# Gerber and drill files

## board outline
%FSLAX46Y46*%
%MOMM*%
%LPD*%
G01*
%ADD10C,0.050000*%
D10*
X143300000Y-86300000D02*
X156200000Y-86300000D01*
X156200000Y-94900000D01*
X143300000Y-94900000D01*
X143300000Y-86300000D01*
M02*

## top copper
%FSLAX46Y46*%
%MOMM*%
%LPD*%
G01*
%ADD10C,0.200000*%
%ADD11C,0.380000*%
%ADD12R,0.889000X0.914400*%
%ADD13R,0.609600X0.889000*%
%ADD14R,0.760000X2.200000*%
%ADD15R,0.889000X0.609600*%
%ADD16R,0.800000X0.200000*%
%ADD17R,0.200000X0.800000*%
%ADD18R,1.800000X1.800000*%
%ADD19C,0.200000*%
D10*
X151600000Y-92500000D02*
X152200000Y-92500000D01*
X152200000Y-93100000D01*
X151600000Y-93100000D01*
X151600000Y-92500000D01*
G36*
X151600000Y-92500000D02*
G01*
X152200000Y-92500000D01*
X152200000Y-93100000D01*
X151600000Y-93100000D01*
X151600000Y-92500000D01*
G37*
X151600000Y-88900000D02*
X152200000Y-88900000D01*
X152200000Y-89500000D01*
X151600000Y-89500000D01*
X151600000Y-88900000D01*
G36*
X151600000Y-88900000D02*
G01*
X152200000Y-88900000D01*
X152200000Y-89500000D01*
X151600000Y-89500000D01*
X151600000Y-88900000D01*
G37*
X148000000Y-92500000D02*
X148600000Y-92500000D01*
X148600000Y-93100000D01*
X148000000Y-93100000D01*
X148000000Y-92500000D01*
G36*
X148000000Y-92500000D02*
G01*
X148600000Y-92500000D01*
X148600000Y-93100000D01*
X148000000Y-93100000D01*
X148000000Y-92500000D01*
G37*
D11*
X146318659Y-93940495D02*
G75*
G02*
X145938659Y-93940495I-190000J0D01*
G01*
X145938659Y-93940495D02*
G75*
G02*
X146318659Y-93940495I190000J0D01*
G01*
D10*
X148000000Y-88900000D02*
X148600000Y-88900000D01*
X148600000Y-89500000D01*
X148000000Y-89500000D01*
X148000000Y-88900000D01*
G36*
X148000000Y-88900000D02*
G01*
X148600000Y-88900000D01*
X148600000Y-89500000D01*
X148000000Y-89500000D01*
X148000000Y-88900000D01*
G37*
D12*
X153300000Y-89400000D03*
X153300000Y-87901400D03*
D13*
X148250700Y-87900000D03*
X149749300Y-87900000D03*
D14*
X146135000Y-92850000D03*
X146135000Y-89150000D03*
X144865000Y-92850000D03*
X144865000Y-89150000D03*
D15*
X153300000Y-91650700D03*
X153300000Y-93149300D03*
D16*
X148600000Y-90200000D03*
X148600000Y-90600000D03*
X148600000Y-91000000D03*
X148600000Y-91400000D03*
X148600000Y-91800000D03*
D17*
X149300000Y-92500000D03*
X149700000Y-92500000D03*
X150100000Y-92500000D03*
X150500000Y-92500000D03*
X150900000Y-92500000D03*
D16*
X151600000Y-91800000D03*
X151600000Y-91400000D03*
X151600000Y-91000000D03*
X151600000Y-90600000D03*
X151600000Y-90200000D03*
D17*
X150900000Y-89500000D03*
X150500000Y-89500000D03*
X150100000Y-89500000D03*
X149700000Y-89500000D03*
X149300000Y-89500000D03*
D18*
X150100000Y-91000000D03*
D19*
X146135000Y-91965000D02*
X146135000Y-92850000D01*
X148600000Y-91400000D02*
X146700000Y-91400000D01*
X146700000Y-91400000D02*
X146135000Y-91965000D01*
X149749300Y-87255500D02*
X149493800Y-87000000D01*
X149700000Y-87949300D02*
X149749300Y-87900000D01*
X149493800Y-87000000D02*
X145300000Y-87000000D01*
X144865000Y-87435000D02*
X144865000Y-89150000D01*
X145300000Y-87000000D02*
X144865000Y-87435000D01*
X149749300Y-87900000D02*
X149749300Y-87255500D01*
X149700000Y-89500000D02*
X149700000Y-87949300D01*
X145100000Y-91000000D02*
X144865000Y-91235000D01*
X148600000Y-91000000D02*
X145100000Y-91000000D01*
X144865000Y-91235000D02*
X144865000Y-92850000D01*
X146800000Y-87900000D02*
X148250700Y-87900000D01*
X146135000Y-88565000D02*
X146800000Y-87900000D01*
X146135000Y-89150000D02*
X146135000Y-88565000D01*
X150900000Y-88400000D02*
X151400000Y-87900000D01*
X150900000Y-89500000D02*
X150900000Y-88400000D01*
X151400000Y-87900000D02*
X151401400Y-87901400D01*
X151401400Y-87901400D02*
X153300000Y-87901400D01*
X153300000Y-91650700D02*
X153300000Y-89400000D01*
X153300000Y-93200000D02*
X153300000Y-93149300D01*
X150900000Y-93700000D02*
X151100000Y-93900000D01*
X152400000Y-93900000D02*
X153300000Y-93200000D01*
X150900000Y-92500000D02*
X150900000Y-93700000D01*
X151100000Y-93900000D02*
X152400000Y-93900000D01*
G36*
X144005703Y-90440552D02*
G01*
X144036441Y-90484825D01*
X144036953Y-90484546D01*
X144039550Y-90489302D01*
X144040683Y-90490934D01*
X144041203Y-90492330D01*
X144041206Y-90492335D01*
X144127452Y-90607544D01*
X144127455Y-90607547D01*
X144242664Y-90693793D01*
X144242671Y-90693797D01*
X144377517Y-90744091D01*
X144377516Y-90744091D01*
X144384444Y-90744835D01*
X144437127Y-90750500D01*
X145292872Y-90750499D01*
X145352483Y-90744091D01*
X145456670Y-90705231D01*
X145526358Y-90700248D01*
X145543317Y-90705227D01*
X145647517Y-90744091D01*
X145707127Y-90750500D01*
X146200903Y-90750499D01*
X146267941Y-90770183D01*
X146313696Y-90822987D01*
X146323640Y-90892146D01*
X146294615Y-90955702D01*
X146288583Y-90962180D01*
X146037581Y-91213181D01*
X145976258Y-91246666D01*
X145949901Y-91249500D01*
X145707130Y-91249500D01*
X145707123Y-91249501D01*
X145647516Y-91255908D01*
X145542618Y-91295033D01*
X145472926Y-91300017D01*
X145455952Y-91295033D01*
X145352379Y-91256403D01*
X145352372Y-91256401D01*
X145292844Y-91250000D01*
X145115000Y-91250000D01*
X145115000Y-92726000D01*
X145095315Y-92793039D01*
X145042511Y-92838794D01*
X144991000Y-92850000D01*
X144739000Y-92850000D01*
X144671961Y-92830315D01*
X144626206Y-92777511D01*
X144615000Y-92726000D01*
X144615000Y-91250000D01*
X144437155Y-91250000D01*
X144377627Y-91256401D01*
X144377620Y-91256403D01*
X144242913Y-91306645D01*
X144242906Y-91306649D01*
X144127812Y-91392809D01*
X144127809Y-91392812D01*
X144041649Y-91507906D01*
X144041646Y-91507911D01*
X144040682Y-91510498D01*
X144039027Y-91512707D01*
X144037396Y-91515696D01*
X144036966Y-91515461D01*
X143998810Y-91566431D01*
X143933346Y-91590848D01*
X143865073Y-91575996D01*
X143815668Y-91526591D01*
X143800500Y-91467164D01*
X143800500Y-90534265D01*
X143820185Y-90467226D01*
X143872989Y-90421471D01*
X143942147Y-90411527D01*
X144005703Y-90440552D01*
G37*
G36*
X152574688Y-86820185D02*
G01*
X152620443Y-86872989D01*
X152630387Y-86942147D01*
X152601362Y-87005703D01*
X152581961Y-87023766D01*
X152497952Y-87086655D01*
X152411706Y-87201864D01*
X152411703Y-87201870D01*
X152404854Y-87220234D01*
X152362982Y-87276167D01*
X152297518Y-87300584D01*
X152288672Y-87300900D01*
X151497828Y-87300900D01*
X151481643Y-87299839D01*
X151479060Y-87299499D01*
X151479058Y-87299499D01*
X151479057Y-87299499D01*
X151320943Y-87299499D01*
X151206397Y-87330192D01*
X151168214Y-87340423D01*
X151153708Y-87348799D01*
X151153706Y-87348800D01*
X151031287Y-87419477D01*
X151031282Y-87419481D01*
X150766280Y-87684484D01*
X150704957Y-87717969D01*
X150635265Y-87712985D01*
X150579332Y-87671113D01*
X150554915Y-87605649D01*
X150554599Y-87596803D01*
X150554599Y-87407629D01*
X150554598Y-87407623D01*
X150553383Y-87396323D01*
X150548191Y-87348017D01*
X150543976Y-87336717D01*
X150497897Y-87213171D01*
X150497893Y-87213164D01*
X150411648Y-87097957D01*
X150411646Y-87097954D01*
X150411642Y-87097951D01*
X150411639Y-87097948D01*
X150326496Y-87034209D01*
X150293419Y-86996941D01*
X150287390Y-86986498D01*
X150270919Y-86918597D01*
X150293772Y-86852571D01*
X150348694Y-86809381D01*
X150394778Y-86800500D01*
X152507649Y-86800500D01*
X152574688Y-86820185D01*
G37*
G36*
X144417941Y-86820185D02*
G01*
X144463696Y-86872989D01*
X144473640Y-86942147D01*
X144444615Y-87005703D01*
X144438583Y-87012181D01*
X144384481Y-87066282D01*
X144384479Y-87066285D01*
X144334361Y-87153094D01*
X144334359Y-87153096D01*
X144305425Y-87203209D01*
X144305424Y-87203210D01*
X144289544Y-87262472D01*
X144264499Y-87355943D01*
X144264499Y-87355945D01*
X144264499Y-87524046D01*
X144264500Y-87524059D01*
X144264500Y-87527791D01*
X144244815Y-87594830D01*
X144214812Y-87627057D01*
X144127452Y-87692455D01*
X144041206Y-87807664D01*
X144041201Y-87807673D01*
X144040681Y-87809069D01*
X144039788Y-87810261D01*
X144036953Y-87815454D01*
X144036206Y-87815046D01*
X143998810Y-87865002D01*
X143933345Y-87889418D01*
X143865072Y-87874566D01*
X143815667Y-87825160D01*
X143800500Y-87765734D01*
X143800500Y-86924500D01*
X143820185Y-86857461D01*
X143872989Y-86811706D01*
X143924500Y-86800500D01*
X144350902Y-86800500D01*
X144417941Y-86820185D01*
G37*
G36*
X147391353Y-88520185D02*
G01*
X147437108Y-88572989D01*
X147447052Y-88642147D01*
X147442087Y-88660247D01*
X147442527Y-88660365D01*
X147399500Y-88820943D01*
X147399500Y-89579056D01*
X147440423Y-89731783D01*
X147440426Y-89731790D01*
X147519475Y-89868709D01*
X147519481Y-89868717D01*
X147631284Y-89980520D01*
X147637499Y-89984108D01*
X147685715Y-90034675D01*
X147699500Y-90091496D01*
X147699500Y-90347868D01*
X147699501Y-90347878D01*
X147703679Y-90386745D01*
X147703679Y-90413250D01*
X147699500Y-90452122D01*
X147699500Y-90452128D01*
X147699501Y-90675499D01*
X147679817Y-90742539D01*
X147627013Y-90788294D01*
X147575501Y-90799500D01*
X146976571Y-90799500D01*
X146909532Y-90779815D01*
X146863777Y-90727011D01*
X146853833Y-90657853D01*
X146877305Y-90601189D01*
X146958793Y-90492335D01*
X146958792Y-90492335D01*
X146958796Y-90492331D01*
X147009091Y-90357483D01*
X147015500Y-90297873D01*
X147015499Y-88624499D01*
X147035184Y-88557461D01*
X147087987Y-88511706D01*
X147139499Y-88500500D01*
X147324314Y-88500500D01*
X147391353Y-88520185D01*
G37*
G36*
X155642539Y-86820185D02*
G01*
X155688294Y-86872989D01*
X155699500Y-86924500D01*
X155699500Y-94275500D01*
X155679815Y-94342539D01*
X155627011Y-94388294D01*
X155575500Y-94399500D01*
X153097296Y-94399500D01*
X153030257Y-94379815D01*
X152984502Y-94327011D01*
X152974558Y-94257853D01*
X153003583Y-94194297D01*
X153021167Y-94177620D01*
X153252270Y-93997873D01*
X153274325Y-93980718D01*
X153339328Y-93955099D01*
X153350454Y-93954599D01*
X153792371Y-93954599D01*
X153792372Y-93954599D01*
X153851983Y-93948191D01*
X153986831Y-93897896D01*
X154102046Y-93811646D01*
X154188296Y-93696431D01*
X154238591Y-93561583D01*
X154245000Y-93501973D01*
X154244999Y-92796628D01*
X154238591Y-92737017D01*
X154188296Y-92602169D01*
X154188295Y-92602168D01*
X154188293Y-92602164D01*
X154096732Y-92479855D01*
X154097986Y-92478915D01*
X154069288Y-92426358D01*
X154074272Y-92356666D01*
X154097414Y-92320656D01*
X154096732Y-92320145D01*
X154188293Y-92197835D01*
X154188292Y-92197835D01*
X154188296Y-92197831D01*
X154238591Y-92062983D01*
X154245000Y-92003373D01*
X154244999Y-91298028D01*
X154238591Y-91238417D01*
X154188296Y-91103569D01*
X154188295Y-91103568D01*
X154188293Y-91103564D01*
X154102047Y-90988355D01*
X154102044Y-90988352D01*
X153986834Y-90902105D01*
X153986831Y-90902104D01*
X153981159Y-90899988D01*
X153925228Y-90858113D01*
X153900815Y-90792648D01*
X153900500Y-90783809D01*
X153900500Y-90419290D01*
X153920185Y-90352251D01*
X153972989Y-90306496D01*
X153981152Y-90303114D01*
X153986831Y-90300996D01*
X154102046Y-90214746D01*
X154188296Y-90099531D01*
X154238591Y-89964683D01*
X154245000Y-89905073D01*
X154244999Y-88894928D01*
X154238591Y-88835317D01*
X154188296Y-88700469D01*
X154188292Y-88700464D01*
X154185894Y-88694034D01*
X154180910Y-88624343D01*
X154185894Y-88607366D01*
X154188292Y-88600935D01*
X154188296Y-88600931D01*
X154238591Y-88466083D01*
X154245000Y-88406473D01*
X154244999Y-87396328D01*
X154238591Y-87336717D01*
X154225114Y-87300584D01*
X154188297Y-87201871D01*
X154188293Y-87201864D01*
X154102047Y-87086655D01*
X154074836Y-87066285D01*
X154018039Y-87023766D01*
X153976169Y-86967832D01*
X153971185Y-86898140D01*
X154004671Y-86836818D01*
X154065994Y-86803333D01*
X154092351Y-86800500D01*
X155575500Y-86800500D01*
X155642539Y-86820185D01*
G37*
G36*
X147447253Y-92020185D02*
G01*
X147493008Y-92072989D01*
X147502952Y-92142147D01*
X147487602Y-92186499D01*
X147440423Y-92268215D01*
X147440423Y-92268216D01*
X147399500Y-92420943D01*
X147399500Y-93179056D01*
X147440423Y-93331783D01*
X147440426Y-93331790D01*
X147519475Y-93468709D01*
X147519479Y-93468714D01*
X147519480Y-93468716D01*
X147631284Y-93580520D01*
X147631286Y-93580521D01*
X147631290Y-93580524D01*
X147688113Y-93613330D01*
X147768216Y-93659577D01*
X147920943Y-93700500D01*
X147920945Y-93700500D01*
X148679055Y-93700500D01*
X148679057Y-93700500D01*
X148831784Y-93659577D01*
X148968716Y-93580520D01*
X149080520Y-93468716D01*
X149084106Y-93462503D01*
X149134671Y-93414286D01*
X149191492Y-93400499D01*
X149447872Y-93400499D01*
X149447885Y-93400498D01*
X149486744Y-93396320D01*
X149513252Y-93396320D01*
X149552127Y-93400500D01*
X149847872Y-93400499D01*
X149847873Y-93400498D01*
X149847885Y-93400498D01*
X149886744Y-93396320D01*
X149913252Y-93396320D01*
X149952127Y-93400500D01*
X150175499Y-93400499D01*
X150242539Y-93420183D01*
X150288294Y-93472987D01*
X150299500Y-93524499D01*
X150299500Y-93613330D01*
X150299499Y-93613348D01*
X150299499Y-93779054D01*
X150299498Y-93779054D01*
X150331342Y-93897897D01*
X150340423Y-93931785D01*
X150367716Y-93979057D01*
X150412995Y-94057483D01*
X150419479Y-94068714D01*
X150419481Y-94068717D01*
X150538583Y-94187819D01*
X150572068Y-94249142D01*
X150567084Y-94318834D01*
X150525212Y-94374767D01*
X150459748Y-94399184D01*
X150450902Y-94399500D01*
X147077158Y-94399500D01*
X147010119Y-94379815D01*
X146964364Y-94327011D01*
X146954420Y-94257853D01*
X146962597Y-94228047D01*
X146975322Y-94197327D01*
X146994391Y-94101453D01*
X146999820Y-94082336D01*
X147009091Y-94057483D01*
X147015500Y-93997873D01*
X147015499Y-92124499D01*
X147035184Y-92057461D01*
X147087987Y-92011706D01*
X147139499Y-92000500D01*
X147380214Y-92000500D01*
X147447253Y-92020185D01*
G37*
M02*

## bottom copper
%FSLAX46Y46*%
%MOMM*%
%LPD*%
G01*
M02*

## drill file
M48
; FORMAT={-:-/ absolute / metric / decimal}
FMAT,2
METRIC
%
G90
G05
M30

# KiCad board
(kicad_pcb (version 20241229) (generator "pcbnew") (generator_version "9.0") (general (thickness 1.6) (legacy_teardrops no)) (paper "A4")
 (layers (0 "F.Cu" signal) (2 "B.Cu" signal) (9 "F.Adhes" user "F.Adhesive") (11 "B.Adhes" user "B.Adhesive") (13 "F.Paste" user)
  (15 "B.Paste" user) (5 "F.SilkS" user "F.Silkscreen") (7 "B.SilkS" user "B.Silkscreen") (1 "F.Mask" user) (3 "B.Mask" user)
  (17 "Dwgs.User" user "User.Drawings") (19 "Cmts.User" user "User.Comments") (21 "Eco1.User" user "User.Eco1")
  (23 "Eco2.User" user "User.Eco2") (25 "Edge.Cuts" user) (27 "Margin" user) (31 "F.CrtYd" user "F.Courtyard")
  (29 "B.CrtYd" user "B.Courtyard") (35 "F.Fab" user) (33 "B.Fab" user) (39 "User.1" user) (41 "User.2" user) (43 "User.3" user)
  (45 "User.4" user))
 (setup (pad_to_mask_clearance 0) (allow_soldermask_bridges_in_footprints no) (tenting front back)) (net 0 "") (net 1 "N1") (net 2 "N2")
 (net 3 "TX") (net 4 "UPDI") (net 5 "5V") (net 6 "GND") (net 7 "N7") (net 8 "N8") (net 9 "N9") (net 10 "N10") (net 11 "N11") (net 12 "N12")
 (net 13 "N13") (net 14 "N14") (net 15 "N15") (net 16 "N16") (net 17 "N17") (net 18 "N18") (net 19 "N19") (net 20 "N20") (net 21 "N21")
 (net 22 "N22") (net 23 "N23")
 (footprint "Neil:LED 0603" (layer "F.Cu") (at 153.3 88.6507 90)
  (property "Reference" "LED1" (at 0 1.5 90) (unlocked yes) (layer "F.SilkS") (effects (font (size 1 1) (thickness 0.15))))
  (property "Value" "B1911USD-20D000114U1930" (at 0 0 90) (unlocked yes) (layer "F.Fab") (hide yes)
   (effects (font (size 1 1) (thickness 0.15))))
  (pad "1" smd rect (at -0.7493 0 90) (size 0.9144 0.889) (layers "F.Cu" "F.Mask" "F.Paste") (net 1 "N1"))
  (pad "2" smd rect (at 0.7493 0 90) (size 0.9144 0.889) (layers "F.Cu" "F.Mask" "F.Paste") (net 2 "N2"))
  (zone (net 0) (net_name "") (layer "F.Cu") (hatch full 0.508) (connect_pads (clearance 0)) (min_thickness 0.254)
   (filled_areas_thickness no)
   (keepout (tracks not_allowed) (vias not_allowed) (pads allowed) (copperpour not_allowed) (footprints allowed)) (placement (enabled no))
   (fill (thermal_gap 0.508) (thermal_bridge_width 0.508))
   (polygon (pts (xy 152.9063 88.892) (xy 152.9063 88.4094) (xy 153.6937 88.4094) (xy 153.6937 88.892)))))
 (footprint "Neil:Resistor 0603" (layer "F.Cu") (at 149 87.9)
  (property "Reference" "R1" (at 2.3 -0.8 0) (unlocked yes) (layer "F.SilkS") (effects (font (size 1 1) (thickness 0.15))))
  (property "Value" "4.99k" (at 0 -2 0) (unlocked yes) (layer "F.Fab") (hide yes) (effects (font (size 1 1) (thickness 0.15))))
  (pad "1" smd rect (at -0.7493 0) (size 0.6096 0.889) (layers "F.Cu" "F.Mask" "F.Paste") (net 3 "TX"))
  (pad "2" smd rect (at 0.7493 0) (size 0.6096 0.889) (layers "F.Cu" "F.Mask" "F.Paste") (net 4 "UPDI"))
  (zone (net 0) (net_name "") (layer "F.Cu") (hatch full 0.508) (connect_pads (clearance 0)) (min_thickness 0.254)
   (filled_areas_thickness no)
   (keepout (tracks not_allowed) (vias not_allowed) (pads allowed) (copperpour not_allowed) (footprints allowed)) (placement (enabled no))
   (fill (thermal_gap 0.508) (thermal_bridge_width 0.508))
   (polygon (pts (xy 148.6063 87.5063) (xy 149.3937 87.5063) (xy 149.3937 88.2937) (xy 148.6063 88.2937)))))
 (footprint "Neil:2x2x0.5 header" (layer "F.Cu") (at 145.5 91 180)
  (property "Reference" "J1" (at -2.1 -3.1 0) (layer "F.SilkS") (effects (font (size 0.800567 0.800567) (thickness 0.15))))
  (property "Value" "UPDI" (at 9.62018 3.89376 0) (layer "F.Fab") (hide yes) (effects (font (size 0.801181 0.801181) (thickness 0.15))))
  (pad "1" smd rect (at -0.635 -1.85 180) (size 0.76 2.2) (layers "F.Cu" "F.Mask" "F.Paste") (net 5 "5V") (solder_mask_margin 0.102))
  (pad "2" smd rect (at -0.635 1.85 180) (size 0.76 2.2) (layers "F.Cu" "F.Mask" "F.Paste") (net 3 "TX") (solder_mask_margin 0.102))
  (pad "3" smd rect (at 0.635 -1.85 180) (size 0.76 2.2) (layers "F.Cu" "F.Mask" "F.Paste") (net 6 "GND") (solder_mask_margin 0.102))
  (pad "4" smd rect (at 0.635 1.85 180) (size 0.76 2.2) (layers "F.Cu" "F.Mask" "F.Paste") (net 4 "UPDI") (solder_mask_margin 0.102)))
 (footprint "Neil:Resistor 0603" (layer "F.Cu") (at 153.3 92.4 -90)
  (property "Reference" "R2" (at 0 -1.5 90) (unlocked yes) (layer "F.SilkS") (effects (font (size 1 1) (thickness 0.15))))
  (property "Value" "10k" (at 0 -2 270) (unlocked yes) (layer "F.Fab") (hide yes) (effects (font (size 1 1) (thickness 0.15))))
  (pad "1" smd rect (at -0.7493 0 270) (size 0.6096 0.889) (layers "F.Cu" "F.Mask" "F.Paste") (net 1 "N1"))
  (pad "2" smd rect (at 0.7493 0 270) (size 0.6096 0.889) (layers "F.Cu" "F.Mask" "F.Paste") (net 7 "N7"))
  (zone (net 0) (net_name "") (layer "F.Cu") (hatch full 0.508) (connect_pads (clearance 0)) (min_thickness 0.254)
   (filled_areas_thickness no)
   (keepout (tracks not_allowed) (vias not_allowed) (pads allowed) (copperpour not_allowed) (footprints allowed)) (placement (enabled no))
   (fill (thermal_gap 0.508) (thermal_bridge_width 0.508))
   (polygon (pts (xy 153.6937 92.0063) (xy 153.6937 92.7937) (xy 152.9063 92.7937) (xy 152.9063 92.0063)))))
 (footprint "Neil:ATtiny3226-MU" (layer "F.Cu") (at 150.1 91)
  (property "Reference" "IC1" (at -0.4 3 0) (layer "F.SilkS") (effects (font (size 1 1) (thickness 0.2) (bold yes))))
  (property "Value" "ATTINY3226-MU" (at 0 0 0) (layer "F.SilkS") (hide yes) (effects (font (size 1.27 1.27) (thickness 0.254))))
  (pad "1" smd rect (at -1.5 -0.8 90) (size 0.2 0.8) (layers "F.Cu" "F.Mask" "F.Paste") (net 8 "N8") (thermal_bridge_angle 45))
  (pad "2" smd rect (at -1.5 -0.4 90) (size 0.2 0.8) (layers "F.Cu" "F.Mask" "F.Paste") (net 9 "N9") (thermal_bridge_angle 45))
  (pad "3" smd rect (at -1.5 0 90) (size 0.2 0.8) (layers "F.Cu" "F.Mask" "F.Paste") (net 6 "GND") (thermal_bridge_angle 45))
  (pad "4" smd rect (at -1.5 0.4 90) (size 0.2 0.8) (layers "F.Cu" "F.Mask" "F.Paste") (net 5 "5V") (thermal_bridge_angle 45))
  (pad "5" smd rect (at -1.5 0.8 90) (size 0.2 0.8) (layers "F.Cu" "F.Mask" "F.Paste") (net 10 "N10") (thermal_bridge_angle 45))
  (pad "6" smd rect (at -0.8 1.5) (size 0.2 0.8) (layers "F.Cu" "F.Mask" "F.Paste") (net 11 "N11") (thermal_bridge_angle 45))
  (pad "7" smd rect (at -0.4 1.5) (size 0.2 0.8) (layers "F.Cu" "F.Mask" "F.Paste") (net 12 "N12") (thermal_bridge_angle 45))
  (pad "8" smd rect (at 0 1.5) (size 0.2 0.8) (layers "F.Cu" "F.Mask" "F.Paste") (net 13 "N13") (thermal_bridge_angle 45))
  (pad "9" smd rect (at 0.4 1.5) (size 0.2 0.8) (layers "F.Cu" "F.Mask" "F.Paste") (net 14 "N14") (thermal_bridge_angle 45))
  (pad "10" smd rect (at 0.8 1.5) (size 0.2 0.8) (layers "F.Cu" "F.Mask" "F.Paste") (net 7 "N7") (thermal_bridge_angle 45))
  (pad "11" smd rect (at 1.5 0.8 90) (size 0.2 0.8) (layers "F.Cu" "F.Mask" "F.Paste") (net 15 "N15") (thermal_bridge_angle 45))
  (pad "12" smd rect (at 1.5 0.4 90) (size 0.2 0.8) (layers "F.Cu" "F.Mask" "F.Paste") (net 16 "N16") (thermal_bridge_angle 45))
  (pad "13" smd rect (at 1.5 0 90) (size 0.2 0.8) (layers "F.Cu" "F.Mask" "F.Paste") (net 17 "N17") (thermal_bridge_angle 45))
  (pad "14" smd rect (at 1.5 -0.4 90) (size 0.2 0.8) (layers "F.Cu" "F.Mask" "F.Paste") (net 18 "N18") (thermal_bridge_angle 45))
  (pad "15" smd rect (at 1.5 -0.8 90) (size 0.2 0.8) (layers "F.Cu" "F.Mask" "F.Paste") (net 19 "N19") (thermal_bridge_angle 45))
  (pad "16" smd rect (at 0.8 -1.5) (size 0.2 0.8) (layers "F.Cu" "F.Mask" "F.Paste") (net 2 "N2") (thermal_bridge_angle 45))
  (pad "17" smd rect (at 0.4 -1.5) (size 0.2 0.8) (layers "F.Cu" "F.Mask" "F.Paste") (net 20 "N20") (thermal_bridge_angle 45))
  (pad "18" smd rect (at 0 -1.5) (size 0.2 0.8) (layers "F.Cu" "F.Mask" "F.Paste") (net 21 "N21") (thermal_bridge_angle 45))
  (pad "19" smd rect (at -0.4 -1.5) (size 0.2 0.8) (layers "F.Cu" "F.Mask" "F.Paste") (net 4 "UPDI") (thermal_bridge_angle 45))
  (pad "20" smd rect (at -0.8 -1.5) (size 0.2 0.8) (layers "F.Cu" "F.Mask" "F.Paste") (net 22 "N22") (thermal_bridge_angle 45))
  (pad "21" smd rect (at 0 0) (size 1.8 1.8) (layers "F.Cu" "F.Mask" "F.Paste") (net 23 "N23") (thermal_bridge_angle 45)))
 (gr_rect (start 151.6 92.5) (end 152.2 93.1) (stroke (width 0.2) (type solid)) (fill yes) (layer "F.Cu"))
 (gr_rect (start 151.6 88.9) (end 152.2 89.5) (stroke (width 0.2) (type solid)) (fill yes) (layer "F.Cu"))
 (gr_rect (start 148 92.5) (end 148.6 93.1) (stroke (width 0.2) (type solid)) (fill yes) (layer "F.Cu"))
 (gr_circle (center 146.128659 93.940495) (end 146.408659 93.940495) (stroke (width 0.2) (type solid)) (fill yes) (layer "F.Cu") (net 5))
 (gr_rect (start 148 88.9) (end 148.6 89.5) (stroke (width 0.2) (type solid)) (fill yes) (layer "F.Cu"))
 (gr_rect (start 143.3 86.3) (end 156.2 94.9) (stroke (width 0.05) (type default)) (fill no) (layer "Edge.Cuts"))
 (segment (start 146.135 91.965) (end 146.135 92.85) (width 0.2) (layer "F.Cu") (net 5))
 (segment (start 148.6 91.4) (end 146.7 91.4) (width 0.2) (layer "F.Cu") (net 5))
 (segment (start 146.7 91.4) (end 146.135 91.965) (width 0.2) (layer "F.Cu") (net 5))
 (segment (start 149.7493 87.2555) (end 149.4938 87) (width 0.2) (layer "F.Cu") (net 4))
 (segment (start 149.7 87.9493) (end 149.7493 87.9) (width 0.2) (layer "F.Cu") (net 4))
 (segment (start 149.4938 87) (end 145.3 87) (width 0.2) (layer "F.Cu") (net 4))
 (segment (start 144.865 87.435) (end 144.865 89.15) (width 0.2) (layer "F.Cu") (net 4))
 (segment (start 145.3 87) (end 144.865 87.435) (width 0.2) (layer "F.Cu") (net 4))
 (segment (start 149.7493 87.9) (end 149.7493 87.2555) (width 0.2) (layer "F.Cu") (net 4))
 (segment (start 149.7 89.5) (end 149.7 87.9493) (width 0.2) (layer "F.Cu") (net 4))
 (segment (start 145.1 91) (end 144.865 91.235) (width 0.2) (layer "F.Cu") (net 6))
 (segment (start 148.6 91) (end 145.1 91) (width 0.2) (layer "F.Cu") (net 6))
 (segment (start 144.865 91.235) (end 144.865 92.85) (width 0.2) (layer "F.Cu") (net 6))
 (segment (start 146.8 87.9) (end 148.2507 87.9) (width 0.2) (layer "F.Cu") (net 3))
 (segment (start 146.135 88.565) (end 146.8 87.9) (width 0.2) (layer "F.Cu") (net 3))
 (segment (start 146.135 89.15) (end 146.135 88.565) (width 0.2) (layer "F.Cu") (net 3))
 (segment (start 150.9 88.4) (end 151.4 87.9) (width 0.2) (layer "F.Cu") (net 2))
 (segment (start 150.9 89.5) (end 150.9 88.4) (width 0.2) (layer "F.Cu") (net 2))
 (segment (start 151.4 87.9) (end 151.4014 87.9014) (width 0.2) (layer "F.Cu") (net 2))
 (segment (start 151.4014 87.9014) (end 153.3 87.9014) (width 0.2) (layer "F.Cu") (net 2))
 (segment (start 153.3 91.6507) (end 153.3 89.4) (width 0.2) (layer "F.Cu") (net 1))
 (segment (start 153.3 93.2) (end 153.3 93.1493) (width 0.2) (layer "F.Cu") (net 7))
 (segment (start 150.9 93.7) (end 151.1 93.9) (width 0.2) (layer "F.Cu") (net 7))
 (segment (start 152.4 93.9) (end 153.3 93.2) (width 0.2) (layer "F.Cu") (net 7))
 (segment (start 150.9 92.5) (end 150.9 93.7) (width 0.2) (layer "F.Cu") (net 7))
 (segment (start 151.1 93.9) (end 152.4 93.9) (width 0.2) (layer "F.Cu") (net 7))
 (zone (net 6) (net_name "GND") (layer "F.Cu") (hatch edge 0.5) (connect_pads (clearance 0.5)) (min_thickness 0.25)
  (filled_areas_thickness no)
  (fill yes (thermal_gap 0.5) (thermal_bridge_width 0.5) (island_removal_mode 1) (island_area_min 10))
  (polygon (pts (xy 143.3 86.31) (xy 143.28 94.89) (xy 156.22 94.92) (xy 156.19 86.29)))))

